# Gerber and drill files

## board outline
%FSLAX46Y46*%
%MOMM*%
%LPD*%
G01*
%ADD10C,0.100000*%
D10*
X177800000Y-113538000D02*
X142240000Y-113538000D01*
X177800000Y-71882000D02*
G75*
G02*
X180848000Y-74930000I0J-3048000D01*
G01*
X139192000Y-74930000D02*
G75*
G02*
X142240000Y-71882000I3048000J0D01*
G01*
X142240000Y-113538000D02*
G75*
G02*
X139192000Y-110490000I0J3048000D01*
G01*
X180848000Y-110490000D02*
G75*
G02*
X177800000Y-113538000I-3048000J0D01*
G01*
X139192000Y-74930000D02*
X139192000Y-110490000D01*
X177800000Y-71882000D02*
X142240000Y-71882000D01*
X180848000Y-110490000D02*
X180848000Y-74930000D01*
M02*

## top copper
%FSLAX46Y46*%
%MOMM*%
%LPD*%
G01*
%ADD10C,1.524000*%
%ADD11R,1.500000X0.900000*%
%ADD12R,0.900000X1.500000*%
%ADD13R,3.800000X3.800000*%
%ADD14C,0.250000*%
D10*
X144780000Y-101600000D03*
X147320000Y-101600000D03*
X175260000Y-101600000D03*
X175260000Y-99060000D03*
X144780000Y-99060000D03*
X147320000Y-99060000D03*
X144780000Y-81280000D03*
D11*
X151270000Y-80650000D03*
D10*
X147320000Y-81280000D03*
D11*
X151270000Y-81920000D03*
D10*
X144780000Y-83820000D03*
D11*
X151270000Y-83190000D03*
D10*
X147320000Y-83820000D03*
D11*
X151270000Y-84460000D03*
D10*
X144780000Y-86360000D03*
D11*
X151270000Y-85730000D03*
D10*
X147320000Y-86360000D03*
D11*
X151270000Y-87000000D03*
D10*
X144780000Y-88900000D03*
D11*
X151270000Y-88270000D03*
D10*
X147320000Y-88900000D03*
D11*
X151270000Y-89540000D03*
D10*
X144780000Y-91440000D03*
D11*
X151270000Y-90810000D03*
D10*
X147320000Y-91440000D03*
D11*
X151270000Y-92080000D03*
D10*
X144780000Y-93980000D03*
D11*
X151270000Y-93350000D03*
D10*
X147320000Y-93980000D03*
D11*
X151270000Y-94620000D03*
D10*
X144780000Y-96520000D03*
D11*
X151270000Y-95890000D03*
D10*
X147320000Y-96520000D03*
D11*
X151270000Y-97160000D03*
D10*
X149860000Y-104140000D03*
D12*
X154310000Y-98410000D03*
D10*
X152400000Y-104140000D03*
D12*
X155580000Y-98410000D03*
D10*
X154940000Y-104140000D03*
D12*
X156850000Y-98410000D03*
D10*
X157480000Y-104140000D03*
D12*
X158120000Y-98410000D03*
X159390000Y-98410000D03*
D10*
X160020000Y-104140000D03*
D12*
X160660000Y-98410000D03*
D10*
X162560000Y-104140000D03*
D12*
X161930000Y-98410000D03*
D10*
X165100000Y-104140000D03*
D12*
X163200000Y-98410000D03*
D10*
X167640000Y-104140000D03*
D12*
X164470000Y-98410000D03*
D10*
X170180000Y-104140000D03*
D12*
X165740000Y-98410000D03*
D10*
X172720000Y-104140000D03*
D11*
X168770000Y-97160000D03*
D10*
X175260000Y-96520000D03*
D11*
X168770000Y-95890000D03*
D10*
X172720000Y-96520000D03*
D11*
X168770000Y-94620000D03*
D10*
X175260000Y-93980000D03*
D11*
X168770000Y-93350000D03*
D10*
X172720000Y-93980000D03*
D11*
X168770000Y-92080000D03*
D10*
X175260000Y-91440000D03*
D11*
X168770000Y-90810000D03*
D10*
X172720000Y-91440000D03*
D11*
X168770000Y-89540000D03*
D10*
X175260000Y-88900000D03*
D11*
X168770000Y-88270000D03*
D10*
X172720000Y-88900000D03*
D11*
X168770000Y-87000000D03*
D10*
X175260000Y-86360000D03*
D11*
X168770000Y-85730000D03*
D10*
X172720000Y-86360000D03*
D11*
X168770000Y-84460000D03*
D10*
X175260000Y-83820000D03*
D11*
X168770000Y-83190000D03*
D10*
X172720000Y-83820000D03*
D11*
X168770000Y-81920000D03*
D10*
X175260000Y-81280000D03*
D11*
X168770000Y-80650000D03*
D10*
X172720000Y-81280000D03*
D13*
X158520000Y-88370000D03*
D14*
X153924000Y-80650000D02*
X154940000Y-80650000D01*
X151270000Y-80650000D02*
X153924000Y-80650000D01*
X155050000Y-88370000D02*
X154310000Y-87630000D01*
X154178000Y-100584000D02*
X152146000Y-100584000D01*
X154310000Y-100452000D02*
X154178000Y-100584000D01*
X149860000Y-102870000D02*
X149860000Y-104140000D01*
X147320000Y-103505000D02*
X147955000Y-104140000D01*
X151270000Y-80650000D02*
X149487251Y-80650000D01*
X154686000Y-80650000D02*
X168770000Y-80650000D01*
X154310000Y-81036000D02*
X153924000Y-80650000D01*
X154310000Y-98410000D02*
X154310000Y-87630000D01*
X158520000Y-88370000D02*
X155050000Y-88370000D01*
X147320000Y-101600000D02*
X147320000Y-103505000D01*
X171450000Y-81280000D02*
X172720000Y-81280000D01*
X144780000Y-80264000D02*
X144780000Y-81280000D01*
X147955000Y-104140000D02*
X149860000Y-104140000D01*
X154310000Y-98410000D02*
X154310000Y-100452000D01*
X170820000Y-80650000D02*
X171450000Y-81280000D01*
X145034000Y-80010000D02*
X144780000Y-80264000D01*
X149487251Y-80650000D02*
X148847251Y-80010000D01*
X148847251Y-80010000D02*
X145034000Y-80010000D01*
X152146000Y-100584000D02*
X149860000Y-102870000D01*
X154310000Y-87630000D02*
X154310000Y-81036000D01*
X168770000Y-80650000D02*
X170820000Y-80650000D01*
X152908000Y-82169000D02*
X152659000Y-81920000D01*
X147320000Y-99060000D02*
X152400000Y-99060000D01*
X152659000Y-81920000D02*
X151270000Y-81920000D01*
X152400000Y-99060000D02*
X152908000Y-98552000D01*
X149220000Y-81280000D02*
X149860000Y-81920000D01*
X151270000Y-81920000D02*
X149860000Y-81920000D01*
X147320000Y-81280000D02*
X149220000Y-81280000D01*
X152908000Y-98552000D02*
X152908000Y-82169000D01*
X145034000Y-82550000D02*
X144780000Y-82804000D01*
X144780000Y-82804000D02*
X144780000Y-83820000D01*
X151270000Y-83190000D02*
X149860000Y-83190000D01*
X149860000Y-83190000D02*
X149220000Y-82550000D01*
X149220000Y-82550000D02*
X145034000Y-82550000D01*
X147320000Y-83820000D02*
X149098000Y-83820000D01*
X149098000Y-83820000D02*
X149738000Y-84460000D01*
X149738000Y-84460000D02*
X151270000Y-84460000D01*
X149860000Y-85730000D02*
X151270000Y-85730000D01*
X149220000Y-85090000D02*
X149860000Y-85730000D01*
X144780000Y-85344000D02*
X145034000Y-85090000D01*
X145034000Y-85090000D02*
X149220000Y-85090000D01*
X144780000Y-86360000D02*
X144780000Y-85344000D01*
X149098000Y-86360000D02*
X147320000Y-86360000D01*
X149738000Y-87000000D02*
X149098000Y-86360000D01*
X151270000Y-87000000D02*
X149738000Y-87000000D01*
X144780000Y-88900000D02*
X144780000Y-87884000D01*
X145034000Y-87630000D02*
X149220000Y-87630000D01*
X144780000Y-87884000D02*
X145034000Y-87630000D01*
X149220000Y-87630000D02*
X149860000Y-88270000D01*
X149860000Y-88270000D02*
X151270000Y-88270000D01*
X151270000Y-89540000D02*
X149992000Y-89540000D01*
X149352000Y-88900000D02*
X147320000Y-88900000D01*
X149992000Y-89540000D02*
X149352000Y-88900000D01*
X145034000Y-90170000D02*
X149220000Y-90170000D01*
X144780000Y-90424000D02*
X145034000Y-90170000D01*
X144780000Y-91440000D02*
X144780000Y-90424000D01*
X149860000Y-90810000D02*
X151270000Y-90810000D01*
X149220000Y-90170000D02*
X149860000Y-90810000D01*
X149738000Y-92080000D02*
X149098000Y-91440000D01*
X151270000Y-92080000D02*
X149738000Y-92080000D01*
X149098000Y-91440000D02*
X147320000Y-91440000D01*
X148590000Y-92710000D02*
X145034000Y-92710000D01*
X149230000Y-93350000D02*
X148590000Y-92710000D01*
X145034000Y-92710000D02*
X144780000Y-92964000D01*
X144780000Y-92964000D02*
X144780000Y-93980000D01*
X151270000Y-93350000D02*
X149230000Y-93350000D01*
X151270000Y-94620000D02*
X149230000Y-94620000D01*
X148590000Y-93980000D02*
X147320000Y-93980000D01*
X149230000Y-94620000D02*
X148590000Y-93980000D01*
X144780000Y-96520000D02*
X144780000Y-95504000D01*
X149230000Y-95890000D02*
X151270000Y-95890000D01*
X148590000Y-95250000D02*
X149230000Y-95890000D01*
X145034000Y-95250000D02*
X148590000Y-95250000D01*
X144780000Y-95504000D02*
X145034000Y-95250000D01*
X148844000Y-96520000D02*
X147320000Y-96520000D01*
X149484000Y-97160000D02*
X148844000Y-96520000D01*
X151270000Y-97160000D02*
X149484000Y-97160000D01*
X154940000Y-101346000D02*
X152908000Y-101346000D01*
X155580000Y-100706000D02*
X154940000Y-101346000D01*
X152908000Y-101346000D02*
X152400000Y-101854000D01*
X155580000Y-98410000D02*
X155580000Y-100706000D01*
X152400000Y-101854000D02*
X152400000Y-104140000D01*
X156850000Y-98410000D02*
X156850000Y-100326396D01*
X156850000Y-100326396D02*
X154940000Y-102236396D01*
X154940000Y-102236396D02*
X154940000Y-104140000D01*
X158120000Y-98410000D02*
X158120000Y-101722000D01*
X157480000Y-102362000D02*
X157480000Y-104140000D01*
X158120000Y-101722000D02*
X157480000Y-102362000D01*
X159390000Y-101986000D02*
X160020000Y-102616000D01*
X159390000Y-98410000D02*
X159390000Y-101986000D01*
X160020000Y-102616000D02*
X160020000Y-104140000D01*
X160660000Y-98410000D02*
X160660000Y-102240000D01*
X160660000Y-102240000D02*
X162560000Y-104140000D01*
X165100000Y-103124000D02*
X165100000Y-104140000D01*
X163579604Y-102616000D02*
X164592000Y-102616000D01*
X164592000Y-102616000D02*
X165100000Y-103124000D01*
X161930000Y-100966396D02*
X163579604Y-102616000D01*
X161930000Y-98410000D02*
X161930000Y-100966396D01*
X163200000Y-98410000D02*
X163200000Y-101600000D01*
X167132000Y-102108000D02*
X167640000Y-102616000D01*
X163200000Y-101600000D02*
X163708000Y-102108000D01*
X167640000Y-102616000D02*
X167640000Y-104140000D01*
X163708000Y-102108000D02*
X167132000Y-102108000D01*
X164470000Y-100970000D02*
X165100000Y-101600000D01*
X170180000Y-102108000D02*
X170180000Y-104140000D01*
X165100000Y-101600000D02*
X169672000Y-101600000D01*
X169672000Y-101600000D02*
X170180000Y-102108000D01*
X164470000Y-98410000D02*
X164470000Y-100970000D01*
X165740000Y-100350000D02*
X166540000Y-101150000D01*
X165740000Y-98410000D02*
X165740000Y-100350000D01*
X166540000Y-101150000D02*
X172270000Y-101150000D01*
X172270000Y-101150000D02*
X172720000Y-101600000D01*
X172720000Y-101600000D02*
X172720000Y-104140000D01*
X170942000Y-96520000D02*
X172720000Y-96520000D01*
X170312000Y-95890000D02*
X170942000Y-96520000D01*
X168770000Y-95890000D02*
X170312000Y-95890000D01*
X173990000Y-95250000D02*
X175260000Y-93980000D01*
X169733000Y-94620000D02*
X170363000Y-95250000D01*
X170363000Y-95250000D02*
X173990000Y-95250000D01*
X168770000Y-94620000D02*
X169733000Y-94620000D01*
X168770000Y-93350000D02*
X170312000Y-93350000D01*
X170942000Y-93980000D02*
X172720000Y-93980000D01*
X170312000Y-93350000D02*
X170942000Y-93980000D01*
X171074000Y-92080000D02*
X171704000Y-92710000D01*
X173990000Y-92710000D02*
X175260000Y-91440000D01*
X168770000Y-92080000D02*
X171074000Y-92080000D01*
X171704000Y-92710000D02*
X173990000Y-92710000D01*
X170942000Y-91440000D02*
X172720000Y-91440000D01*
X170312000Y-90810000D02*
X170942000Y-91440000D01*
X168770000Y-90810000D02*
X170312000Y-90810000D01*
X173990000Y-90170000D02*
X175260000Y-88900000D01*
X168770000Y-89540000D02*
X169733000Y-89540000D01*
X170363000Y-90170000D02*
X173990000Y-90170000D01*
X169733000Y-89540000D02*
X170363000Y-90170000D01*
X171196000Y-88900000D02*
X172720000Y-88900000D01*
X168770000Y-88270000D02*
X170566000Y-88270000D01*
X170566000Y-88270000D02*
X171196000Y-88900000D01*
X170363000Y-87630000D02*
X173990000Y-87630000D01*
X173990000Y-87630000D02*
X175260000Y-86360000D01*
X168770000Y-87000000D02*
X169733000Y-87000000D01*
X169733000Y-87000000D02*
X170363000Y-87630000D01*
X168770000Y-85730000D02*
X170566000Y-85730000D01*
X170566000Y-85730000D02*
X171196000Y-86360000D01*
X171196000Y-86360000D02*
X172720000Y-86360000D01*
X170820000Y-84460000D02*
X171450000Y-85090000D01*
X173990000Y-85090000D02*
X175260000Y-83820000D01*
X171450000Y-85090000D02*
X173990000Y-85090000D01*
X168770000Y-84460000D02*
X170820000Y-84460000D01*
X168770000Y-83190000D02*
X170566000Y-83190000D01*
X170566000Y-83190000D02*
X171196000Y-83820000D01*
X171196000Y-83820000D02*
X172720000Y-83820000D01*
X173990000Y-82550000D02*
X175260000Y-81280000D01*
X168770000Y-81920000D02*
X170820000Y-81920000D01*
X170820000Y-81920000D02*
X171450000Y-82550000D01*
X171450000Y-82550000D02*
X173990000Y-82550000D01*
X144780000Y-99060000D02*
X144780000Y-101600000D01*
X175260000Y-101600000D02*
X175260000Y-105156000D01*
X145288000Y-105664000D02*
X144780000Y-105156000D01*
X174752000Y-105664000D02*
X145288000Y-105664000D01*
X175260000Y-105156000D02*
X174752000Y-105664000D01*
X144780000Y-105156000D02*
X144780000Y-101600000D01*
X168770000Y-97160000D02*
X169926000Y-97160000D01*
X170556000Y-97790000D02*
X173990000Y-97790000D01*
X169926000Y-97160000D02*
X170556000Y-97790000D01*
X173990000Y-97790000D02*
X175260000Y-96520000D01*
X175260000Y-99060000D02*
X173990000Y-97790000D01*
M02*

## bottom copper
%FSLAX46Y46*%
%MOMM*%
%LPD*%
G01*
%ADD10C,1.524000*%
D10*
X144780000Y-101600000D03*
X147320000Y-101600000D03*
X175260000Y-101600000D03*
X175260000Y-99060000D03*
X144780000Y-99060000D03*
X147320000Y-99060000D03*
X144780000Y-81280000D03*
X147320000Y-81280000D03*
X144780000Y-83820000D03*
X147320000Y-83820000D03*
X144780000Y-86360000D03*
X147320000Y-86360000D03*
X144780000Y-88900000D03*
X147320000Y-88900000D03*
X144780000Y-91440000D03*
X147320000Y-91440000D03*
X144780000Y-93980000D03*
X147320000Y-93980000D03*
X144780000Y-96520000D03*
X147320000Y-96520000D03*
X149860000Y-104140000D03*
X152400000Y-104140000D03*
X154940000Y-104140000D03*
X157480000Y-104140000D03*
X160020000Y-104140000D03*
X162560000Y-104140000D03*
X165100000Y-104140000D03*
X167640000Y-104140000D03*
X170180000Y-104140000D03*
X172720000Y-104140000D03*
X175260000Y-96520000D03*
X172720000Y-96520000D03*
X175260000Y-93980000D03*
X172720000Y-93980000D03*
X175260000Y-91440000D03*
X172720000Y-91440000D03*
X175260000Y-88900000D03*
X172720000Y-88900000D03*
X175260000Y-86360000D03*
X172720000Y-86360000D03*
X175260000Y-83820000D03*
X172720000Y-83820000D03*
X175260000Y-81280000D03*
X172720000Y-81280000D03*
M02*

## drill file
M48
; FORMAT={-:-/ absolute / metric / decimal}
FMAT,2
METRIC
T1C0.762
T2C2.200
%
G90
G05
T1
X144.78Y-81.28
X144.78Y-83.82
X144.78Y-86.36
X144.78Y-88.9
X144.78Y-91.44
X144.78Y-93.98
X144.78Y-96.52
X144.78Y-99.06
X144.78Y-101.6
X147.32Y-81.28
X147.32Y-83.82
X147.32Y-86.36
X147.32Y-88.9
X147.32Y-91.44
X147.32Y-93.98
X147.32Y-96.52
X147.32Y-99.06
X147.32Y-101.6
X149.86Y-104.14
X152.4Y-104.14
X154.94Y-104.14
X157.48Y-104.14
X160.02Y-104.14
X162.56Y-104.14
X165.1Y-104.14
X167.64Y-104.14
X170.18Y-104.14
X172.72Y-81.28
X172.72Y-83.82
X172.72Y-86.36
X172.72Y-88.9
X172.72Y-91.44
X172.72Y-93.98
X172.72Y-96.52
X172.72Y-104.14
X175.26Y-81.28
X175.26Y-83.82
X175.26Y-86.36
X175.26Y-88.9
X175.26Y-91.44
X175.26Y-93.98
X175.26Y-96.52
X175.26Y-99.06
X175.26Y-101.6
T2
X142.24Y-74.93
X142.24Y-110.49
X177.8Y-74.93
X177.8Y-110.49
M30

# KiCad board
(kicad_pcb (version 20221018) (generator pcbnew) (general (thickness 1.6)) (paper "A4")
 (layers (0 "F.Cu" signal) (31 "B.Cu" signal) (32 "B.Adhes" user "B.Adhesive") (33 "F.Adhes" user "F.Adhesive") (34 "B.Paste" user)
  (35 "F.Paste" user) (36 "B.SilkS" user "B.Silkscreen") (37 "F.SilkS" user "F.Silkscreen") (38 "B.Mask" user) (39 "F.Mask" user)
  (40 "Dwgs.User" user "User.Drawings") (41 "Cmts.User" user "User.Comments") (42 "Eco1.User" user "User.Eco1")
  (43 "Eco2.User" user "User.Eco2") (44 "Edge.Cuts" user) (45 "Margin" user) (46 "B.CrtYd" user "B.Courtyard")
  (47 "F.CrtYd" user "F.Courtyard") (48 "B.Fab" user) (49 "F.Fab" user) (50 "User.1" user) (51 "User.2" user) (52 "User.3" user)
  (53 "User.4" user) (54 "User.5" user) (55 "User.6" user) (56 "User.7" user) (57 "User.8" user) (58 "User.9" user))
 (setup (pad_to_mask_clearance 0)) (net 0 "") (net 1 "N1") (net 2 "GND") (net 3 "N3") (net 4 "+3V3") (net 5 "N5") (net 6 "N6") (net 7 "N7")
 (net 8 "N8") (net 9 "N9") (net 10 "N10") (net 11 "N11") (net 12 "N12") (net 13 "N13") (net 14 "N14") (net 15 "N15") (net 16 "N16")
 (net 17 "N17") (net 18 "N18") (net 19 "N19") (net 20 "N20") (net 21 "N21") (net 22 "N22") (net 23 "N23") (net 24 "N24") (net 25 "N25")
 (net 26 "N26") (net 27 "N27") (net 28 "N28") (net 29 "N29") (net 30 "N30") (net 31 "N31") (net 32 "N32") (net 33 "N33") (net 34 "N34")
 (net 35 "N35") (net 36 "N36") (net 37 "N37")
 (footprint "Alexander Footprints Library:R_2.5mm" (layer "F.Cu") (at 147.32 104.14)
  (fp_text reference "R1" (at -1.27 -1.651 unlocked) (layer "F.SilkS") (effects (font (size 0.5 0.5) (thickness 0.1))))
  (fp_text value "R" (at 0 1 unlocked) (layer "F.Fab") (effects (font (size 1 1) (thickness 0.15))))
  (pad "1" thru_hole circle (at -2.54 -2.54) (size 1.524 1.524) (drill 0.762) (layers "*.Cu" "*.Mask") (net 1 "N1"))
  (pad "2" thru_hole circle (at 0 -2.54) (size 1.524 1.524) (drill 0.762) (layers "*.Cu" "*.Mask") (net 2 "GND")))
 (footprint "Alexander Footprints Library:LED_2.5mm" (layer "F.Cu") (at 177.8 99.06 90)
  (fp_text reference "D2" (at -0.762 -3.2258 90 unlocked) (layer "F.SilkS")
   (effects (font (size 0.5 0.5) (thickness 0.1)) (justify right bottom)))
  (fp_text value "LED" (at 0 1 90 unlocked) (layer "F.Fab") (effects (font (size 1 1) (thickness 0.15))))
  (pad "1" thru_hole circle (at -2.54 -2.54 90) (size 1.524 1.524) (drill 0.762) (layers "*.Cu" "*.Mask") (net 1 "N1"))
  (pad "2" thru_hole circle (at 0 -2.54 90) (size 1.524 1.524) (drill 0.762) (layers "*.Cu" "*.Mask") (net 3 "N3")))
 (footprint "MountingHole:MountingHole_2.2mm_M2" (layer "F.Cu") (at 142.24 74.93)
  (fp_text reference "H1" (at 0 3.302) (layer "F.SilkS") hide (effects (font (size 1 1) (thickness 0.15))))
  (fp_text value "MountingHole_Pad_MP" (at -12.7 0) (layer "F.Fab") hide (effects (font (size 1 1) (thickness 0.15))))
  (pad "" np_thru_hole circle (at 0 0) (size 2.2 2.2) (drill 2.2) (layers "*.Cu" "*.Mask")))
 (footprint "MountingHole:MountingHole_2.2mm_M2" (layer "F.Cu") (at 142.24 110.49)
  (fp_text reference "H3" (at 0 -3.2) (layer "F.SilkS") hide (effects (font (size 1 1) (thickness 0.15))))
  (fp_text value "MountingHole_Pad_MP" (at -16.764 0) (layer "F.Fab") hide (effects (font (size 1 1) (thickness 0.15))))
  (pad "" np_thru_hole circle (at 0 0) (size 2.2 2.2) (drill 2.2) (layers "*.Cu" "*.Mask")))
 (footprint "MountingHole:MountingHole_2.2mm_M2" (layer "F.Cu") (at 177.8 110.49)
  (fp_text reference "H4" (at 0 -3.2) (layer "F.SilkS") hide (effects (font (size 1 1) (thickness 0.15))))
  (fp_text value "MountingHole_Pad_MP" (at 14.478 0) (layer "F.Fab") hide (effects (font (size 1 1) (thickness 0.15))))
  (pad "" np_thru_hole circle (at 0 0) (size 2.2 2.2) (drill 2.2) (layers "*.Cu" "*.Mask")))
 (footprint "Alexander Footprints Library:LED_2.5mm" (layer "F.Cu") (at 147.32 109.22)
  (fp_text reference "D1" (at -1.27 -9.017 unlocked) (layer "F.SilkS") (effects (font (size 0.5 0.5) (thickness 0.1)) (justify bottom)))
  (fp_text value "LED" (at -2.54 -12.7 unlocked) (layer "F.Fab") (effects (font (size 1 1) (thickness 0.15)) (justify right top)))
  (pad "1" thru_hole circle (at -2.54 -10.16) (size 1.524 1.524) (drill 0.762) (layers "*.Cu" "*.Mask") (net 1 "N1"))
  (pad "2" thru_hole circle (at 0 -10.16) (size 1.524 1.524) (drill 0.762) (layers "*.Cu" "*.Mask") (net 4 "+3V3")))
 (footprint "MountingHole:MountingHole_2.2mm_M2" (layer "F.Cu") (at 177.8 74.93)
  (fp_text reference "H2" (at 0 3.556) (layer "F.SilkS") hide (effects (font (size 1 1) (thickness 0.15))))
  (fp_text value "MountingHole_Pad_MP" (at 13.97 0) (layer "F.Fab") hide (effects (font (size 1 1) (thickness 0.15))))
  (pad "" np_thru_hole circle (at 0 0) (size 2.2 2.2) (drill 2.2) (layers "*.Cu" "*.Mask")))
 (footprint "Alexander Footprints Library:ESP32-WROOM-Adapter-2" (layer "F.Cu") (at 160.02 88.9)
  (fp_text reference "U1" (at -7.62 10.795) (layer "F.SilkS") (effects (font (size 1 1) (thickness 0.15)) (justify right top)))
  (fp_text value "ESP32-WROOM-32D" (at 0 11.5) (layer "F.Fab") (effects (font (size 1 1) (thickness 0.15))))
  (pad "1" thru_hole circle (at -15.24 -7.62) (size 1.524 1.524) (drill 0.762) (layers "*.Cu" "*.Mask") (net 2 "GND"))
  (pad "1" smd rect (at -8.75 -8.25) (size 1.5 0.9) (layers "F.Cu" "F.Paste" "F.Mask") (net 2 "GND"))
  (pad "2" thru_hole circle (at -12.7 -7.62) (size 1.524 1.524) (drill 0.762) (layers "*.Cu" "*.Mask") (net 4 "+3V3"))
  (pad "2" smd rect (at -8.75 -6.98) (size 1.5 0.9) (layers "F.Cu" "F.Paste" "F.Mask") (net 4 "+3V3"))
  (pad "3" thru_hole circle (at -15.24 -5.08) (size 1.524 1.524) (drill 0.762) (layers "*.Cu" "*.Mask") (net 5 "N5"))
  (pad "3" smd rect (at -8.75 -5.71) (size 1.5 0.9) (layers "F.Cu" "F.Paste" "F.Mask") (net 5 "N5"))
  (pad "4" thru_hole circle (at -12.7 -5.08) (size 1.524 1.524) (drill 0.762) (layers "*.Cu" "*.Mask") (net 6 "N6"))
  (pad "4" smd rect (at -8.75 -4.44) (size 1.5 0.9) (layers "F.Cu" "F.Paste" "F.Mask") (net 6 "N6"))
  (pad "5" thru_hole circle (at -15.24 -2.54) (size 1.524 1.524) (drill 0.762) (layers "*.Cu" "*.Mask") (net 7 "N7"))
  (pad "5" smd rect (at -8.75 -3.17) (size 1.5 0.9) (layers "F.Cu" "F.Paste" "F.Mask") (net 7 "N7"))
  (pad "6" thru_hole circle (at -12.7 -2.54) (size 1.524 1.524) (drill 0.762) (layers "*.Cu" "*.Mask") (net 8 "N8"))
  (pad "6" smd rect (at -8.75 -1.9) (size 1.5 0.9) (layers "F.Cu" "F.Paste" "F.Mask") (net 8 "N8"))
  (pad "7" thru_hole circle (at -15.24 0) (size 1.524 1.524) (drill 0.762) (layers "*.Cu" "*.Mask") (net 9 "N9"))
  (pad "7" smd rect (at -8.75 -0.63) (size 1.5 0.9) (layers "F.Cu" "F.Paste" "F.Mask") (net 9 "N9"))
  (pad "8" thru_hole circle (at -12.7 0) (size 1.524 1.524) (drill 0.762) (layers "*.Cu" "*.Mask") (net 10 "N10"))
  (pad "8" smd rect (at -8.75 0.64) (size 1.5 0.9) (layers "F.Cu" "F.Paste" "F.Mask") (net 10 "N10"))
  (pad "9" thru_hole circle (at -15.24 2.54) (size 1.524 1.524) (drill 0.762) (layers "*.Cu" "*.Mask") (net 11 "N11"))
  (pad "9" smd rect (at -8.75 1.91) (size 1.5 0.9) (layers "F.Cu" "F.Paste" "F.Mask") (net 11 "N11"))
  (pad "10" thru_hole circle (at -12.7 2.54) (size 1.524 1.524) (drill 0.762) (layers "*.Cu" "*.Mask") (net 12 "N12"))
  (pad "10" smd rect (at -8.75 3.18) (size 1.5 0.9) (layers "F.Cu" "F.Paste" "F.Mask") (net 12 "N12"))
  (pad "11" thru_hole circle (at -15.24 5.08) (size 1.524 1.524) (drill 0.762) (layers "*.Cu" "*.Mask") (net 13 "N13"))
  (pad "11" smd rect (at -8.75 4.45) (size 1.5 0.9) (layers "F.Cu" "F.Paste" "F.Mask") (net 13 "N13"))
  (pad "12" thru_hole circle (at -12.7 5.08) (size 1.524 1.524) (drill 0.762) (layers "*.Cu" "*.Mask") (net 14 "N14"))
  (pad "12" smd rect (at -8.75 5.72) (size 1.5 0.9) (layers "F.Cu" "F.Paste" "F.Mask") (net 14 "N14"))
  (pad "13" thru_hole circle (at -15.24 7.62) (size 1.524 1.524) (drill 0.762) (layers "*.Cu" "*.Mask") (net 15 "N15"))
  (pad "13" smd rect (at -8.75 6.99) (size 1.5 0.9) (layers "F.Cu" "F.Paste" "F.Mask") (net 15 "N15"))
  (pad "14" thru_hole circle (at -12.7 7.62) (size 1.524 1.524) (drill 0.762) (layers "*.Cu" "*.Mask") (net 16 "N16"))
  (pad "14" smd rect (at -8.75 8.26) (size 1.5 0.9) (layers "F.Cu" "F.Paste" "F.Mask") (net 16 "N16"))
  (pad "15" thru_hole circle (at -10.16 15.24 90) (size 1.524 1.524) (drill 0.762) (layers "*.Cu" "*.Mask") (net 2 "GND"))
  (pad "15" smd rect (at -5.71 9.51 90) (size 1.5 0.9) (layers "F.Cu" "F.Paste" "F.Mask") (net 2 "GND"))
  (pad "16" thru_hole circle (at -7.62 15.24 90) (size 1.524 1.524) (drill 0.762) (layers "*.Cu" "*.Mask") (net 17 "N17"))
  (pad "16" smd rect (at -4.44 9.51 90) (size 1.5 0.9) (layers "F.Cu" "F.Paste" "F.Mask") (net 17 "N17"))
  (pad "17" thru_hole circle (at -5.08 15.24 90) (size 1.524 1.524) (drill 0.762) (layers "*.Cu" "*.Mask") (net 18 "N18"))
  (pad "17" smd rect (at -3.17 9.51 90) (size 1.5 0.9) (layers "F.Cu" "F.Paste" "F.Mask") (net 18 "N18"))
  (pad "18" thru_hole circle (at -2.54 15.24 90) (size 1.524 1.524) (drill 0.762) (layers "*.Cu" "*.Mask") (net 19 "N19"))
  (pad "18" smd rect (at -1.9 9.51 90) (size 1.5 0.9) (layers "F.Cu" "F.Paste" "F.Mask") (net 19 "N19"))
  (pad "19" smd rect (at -0.63 9.51 90) (size 1.5 0.9) (layers "F.Cu" "F.Paste" "F.Mask") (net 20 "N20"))
  (pad "19" thru_hole circle (at 0 15.24 90) (size 1.524 1.524) (drill 0.762) (layers "*.Cu" "*.Mask") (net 20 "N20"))
  (pad "20" smd rect (at 0.64 9.51 90) (size 1.5 0.9) (layers "F.Cu" "F.Paste" "F.Mask") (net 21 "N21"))
  (pad "20" thru_hole circle (at 2.54 15.24 90) (size 1.524 1.524) (drill 0.762) (layers "*.Cu" "*.Mask") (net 21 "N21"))
  (pad "21" smd rect (at 1.91 9.51 90) (size 1.5 0.9) (layers "F.Cu" "F.Paste" "F.Mask") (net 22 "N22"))
  (pad "21" thru_hole circle (at 5.08 15.24 90) (size 1.524 1.524) (drill 0.762) (layers "*.Cu" "*.Mask") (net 22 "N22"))
  (pad "22" smd rect (at 3.18 9.51 90) (size 1.5 0.9) (layers "F.Cu" "F.Paste" "F.Mask") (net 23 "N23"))
  (pad "22" thru_hole circle (at 7.62 15.24 90) (size 1.524 1.524) (drill 0.762) (layers "*.Cu" "*.Mask") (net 23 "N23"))
  (pad "23" smd rect (at 4.45 9.51 90) (size 1.5 0.9) (layers "F.Cu" "F.Paste" "F.Mask") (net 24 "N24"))
  (pad "23" thru_hole circle (at 10.16 15.24 90) (size 1.524 1.524) (drill 0.762) (layers "*.Cu" "*.Mask") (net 24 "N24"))
  (pad "24" smd rect (at 5.72 9.51 90) (size 1.5 0.9) (layers "F.Cu" "F.Paste" "F.Mask") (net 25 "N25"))
  (pad "24" thru_hole circle (at 12.7 15.24 90) (size 1.524 1.524) (drill 0.762) (layers "*.Cu" "*.Mask") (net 25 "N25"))
  (pad "25" smd rect (at 8.75 8.26) (size 1.5 0.9) (layers "F.Cu" "F.Paste" "F.Mask") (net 3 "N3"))
  (pad "25" thru_hole circle (at 15.24 7.62) (size 1.524 1.524) (drill 0.762) (layers "*.Cu" "*.Mask") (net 3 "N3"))
  (pad "26" smd rect (at 8.75 6.99) (size 1.5 0.9) (layers "F.Cu" "F.Paste" "F.Mask") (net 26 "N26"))
  (pad "26" thru_hole circle (at 12.7 7.62) (size 1.524 1.524) (drill 0.762) (layers "*.Cu" "*.Mask") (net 26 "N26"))
  (pad "27" smd rect (at 8.75 5.72) (size 1.5 0.9) (layers "F.Cu" "F.Paste" "F.Mask") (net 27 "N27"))
  (pad "27" thru_hole circle (at 15.24 5.08) (size 1.524 1.524) (drill 0.762) (layers "*.Cu" "*.Mask") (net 27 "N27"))
  (pad "28" smd rect (at 8.75 4.45) (size 1.5 0.9) (layers "F.Cu" "F.Paste" "F.Mask") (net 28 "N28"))
  (pad "28" thru_hole circle (at 12.7 5.08) (size 1.524 1.524) (drill 0.762) (layers "*.Cu" "*.Mask") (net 28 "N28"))
  (pad "29" smd rect (at 8.75 3.18) (size 1.5 0.9) (layers "F.Cu" "F.Paste" "F.Mask") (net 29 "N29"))
  (pad "29" thru_hole circle (at 15.24 2.54) (size 1.524 1.524) (drill 0.762) (layers "*.Cu" "*.Mask") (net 29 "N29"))
  (pad "30" smd rect (at 8.75 1.91) (size 1.5 0.9) (layers "F.Cu" "F.Paste" "F.Mask") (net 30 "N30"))
  (pad "30" thru_hole circle (at 12.7 2.54) (size 1.524 1.524) (drill 0.762) (layers "*.Cu" "*.Mask") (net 30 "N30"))
  (pad "31" smd rect (at 8.75 0.64) (size 1.5 0.9) (layers "F.Cu" "F.Paste" "F.Mask") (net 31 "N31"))
  (pad "31" thru_hole circle (at 15.24 0) (size 1.524 1.524) (drill 0.762) (layers "*.Cu" "*.Mask") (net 31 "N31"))
  (pad "32" smd rect (at 8.75 -0.63) (size 1.5 0.9) (layers "F.Cu" "F.Paste" "F.Mask") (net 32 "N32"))
  (pad "32" thru_hole circle (at 12.7 0) (size 1.524 1.524) (drill 0.762) (layers "*.Cu" "*.Mask") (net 32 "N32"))
  (pad "33" smd rect (at 8.75 -1.9) (size 1.5 0.9) (layers "F.Cu" "F.Paste" "F.Mask") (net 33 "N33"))
  (pad "33" thru_hole circle (at 15.24 -2.54) (size 1.524 1.524) (drill 0.762) (layers "*.Cu" "*.Mask") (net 33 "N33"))
  (pad "34" smd rect (at 8.75 -3.17) (size 1.5 0.9) (layers "F.Cu" "F.Paste" "F.Mask") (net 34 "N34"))
  (pad "34" thru_hole circle (at 12.7 -2.54) (size 1.524 1.524) (drill 0.762) (layers "*.Cu" "*.Mask") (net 34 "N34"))
  (pad "35" smd rect (at 8.75 -4.44) (size 1.5 0.9) (layers "F.Cu" "F.Paste" "F.Mask") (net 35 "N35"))
  (pad "35" thru_hole circle (at 15.24 -5.08) (size 1.524 1.524) (drill 0.762) (layers "*.Cu" "*.Mask") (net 35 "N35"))
  (pad "36" smd rect (at 8.75 -5.71) (size 1.5 0.9) (layers "F.Cu" "F.Paste" "F.Mask") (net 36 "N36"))
  (pad "36" thru_hole circle (at 12.7 -5.08) (size 1.524 1.524) (drill 0.762) (layers "*.Cu" "*.Mask") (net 36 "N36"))
  (pad "37" smd rect (at 8.75 -6.98) (size 1.5 0.9) (layers "F.Cu" "F.Paste" "F.Mask") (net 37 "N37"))
  (pad "37" thru_hole circle (at 15.24 -7.62) (size 1.524 1.524) (drill 0.762) (layers "*.Cu" "*.Mask") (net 37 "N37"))
  (pad "38" smd rect (at 8.75 -8.25) (size 1.5 0.9) (layers "F.Cu" "F.Paste" "F.Mask") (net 2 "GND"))
  (pad "38" thru_hole circle (at 12.7 -7.62) (size 1.524 1.524) (drill 0.762) (layers "*.Cu" "*.Mask") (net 2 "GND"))
  (pad "39" smd rect (at -1.5 -0.53) (size 3.8 3.8) (layers "F.Cu" "F.Mask") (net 2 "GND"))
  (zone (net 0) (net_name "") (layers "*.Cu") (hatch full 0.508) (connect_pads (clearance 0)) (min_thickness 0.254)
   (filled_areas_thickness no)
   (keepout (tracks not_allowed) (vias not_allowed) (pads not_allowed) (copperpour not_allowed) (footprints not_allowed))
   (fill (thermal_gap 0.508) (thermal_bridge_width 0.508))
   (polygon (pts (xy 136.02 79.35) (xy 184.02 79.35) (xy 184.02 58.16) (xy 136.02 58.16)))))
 (gr_line (start 177.8 113.538) (end 142.24 113.538) (stroke (width 0.1) (type default)) (layer "Edge.Cuts"))
 (gr_arc (start 177.8 71.882) (mid 179.955261 72.774739) (end 180.848 74.93) (stroke (width 0.1) (type default)) (layer "Edge.Cuts"))
 (gr_arc (start 139.192 74.93) (mid 140.084739 72.774739) (end 142.24 71.882) (stroke (width 0.1) (type default)) (layer "Edge.Cuts"))
 (gr_arc (start 142.24 113.538) (mid 140.084739 112.645261) (end 139.192 110.49) (stroke (width 0.1) (type default)) (layer "Edge.Cuts"))
 (gr_arc (start 180.848 110.49) (mid 179.955261 112.645261) (end 177.8 113.538) (stroke (width 0.1) (type default)) (layer "Edge.Cuts"))
 (gr_line (start 139.192 74.93) (end 139.192 110.49) (stroke (width 0.1) (type default)) (layer "Edge.Cuts"))
 (gr_line (start 177.8 71.882) (end 142.24 71.882) (stroke (width 0.1) (type default)) (layer "Edge.Cuts"))
 (gr_line (start 180.848 110.49) (end 180.848 74.93) (stroke (width 0.1) (type default)) (layer "Edge.Cuts"))
 (segment (start 153.924 80.65) (end 154.94 80.65) (width 0.25) (layer "F.Cu") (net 2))
 (segment (start 151.27 80.65) (end 153.924 80.65) (width 0.25) (layer "F.Cu") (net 2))
 (segment (start 155.05 88.37) (end 154.31 87.63) (width 0.25) (layer "F.Cu") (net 2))
 (segment (start 154.178 100.584) (end 152.146 100.584) (width 0.25) (layer "F.Cu") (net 2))
 (segment (start 154.31 100.452) (end 154.178 100.584) (width 0.25) (layer "F.Cu") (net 2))
 (segment (start 149.86 102.87) (end 149.86 104.14) (width 0.25) (layer "F.Cu") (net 2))
 (segment (start 147.32 103.505) (end 147.955 104.14) (width 0.25) (layer "F.Cu") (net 2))
 (segment (start 151.27 80.65) (end 149.487251 80.65) (width 0.25) (layer "F.Cu") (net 2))
 (segment (start 154.686 80.65) (end 168.77 80.65) (width 0.25) (layer "F.Cu") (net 2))
 (segment (start 154.31 81.036) (end 153.924 80.65) (width 0.25) (layer "F.Cu") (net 2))
 (segment (start 154.31 98.41) (end 154.31 87.63) (width 0.25) (layer "F.Cu") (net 2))
 (segment (start 158.52 88.37) (end 155.05 88.37) (width 0.25) (layer "F.Cu") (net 2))
 (segment (start 147.32 101.6) (end 147.32 103.505) (width 0.25) (layer "F.Cu") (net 2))
 (segment (start 171.45 81.28) (end 172.72 81.28) (width 0.25) (layer "F.Cu") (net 2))
 (segment (start 144.78 80.264) (end 144.78 81.28) (width 0.25) (layer "F.Cu") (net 2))
 (segment (start 147.955 104.14) (end 149.86 104.14) (width 0.25) (layer "F.Cu") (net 2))
 (segment (start 154.31 98.41) (end 154.31 100.452) (width 0.25) (layer "F.Cu") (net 2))
 (segment (start 170.82 80.65) (end 171.45 81.28) (width 0.25) (layer "F.Cu") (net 2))
 (segment (start 145.034 80.01) (end 144.78 80.264) (width 0.25) (layer "F.Cu") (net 2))
 (segment (start 149.487251 80.65) (end 148.847251 80.01) (width 0.25) (layer "F.Cu") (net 2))
 (segment (start 148.847251 80.01) (end 145.034 80.01) (width 0.25) (layer "F.Cu") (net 2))
 (segment (start 152.146 100.584) (end 149.86 102.87) (width 0.25) (layer "F.Cu") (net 2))
 (segment (start 154.31 87.63) (end 154.31 81.036) (width 0.25) (layer "F.Cu") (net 2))
 (segment (start 168.77 80.65) (end 170.82 80.65) (width 0.25) (layer "F.Cu") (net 2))
 (segment (start 152.908 82.169) (end 152.659 81.92) (width 0.25) (layer "F.Cu") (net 4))
 (segment (start 147.32 99.06) (end 152.4 99.06) (width 0.25) (layer "F.Cu") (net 4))
 (segment (start 152.659 81.92) (end 151.27 81.92) (width 0.25) (layer "F.Cu") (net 4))
 (segment (start 152.4 99.06) (end 152.908 98.552) (width 0.25) (layer "F.Cu") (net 4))
 (segment (start 149.22 81.28) (end 149.86 81.92) (width 0.25) (layer "F.Cu") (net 4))
 (segment (start 151.27 81.92) (end 149.86 81.92) (width 0.25) (layer "F.Cu") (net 4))
 (segment (start 147.32 81.28) (end 149.22 81.28) (width 0.25) (layer "F.Cu") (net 4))
 (segment (start 152.908 98.552) (end 152.908 82.169) (width 0.25) (layer "F.Cu") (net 4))
 (segment (start 145.034 82.55) (end 144.78 82.804) (width 0.25) (layer "F.Cu") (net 5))
 (segment (start 144.78 82.804) (end 144.78 83.82) (width 0.25) (layer "F.Cu") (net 5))
 (segment (start 151.27 83.19) (end 149.86 83.19) (width 0.25) (layer "F.Cu") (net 5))
 (segment (start 149.86 83.19) (end 149.22 82.55) (width 0.25) (layer "F.Cu") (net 5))
 (segment (start 149.22 82.55) (end 145.034 82.55) (width 0.25) (layer "F.Cu") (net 5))
 (segment (start 147.32 83.82) (end 149.098 83.82) (width 0.25) (layer "F.Cu") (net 6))
 (segment (start 149.098 83.82) (end 149.738 84.46) (width 0.25) (layer "F.Cu") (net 6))
 (segment (start 149.738 84.46) (end 151.27 84.46) (width 0.25) (layer "F.Cu") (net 6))
 (segment (start 149.86 85.73) (end 151.27 85.73) (width 0.25) (layer "F.Cu") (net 7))
 (segment (start 149.22 85.09) (end 149.86 85.73) (width 0.25) (layer "F.Cu") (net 7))
 (segment (start 144.78 85.344) (end 145.034 85.09) (width 0.25) (layer "F.Cu") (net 7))
 (segment (start 145.034 85.09) (end 149.22 85.09) (width 0.25) (layer "F.Cu") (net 7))
 (segment (start 144.78 86.36) (end 144.78 85.344) (width 0.25) (layer "F.Cu") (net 7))
 (segment (start 149.098 86.36) (end 147.32 86.36) (width 0.25) (layer "F.Cu") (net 8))
 (segment (start 149.738 87) (end 149.098 86.36) (width 0.25) (layer "F.Cu") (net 8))
 (segment (start 151.27 87) (end 149.738 87) (width 0.25) (layer "F.Cu") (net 8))
 (segment (start 144.78 88.9) (end 144.78 87.884) (width 0.25) (layer "F.Cu") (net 9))
 (segment (start 145.034 87.63) (end 149.22 87.63) (width 0.25) (layer "F.Cu") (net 9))
 (segment (start 144.78 87.884) (end 145.034 87.63) (width 0.25) (layer "F.Cu") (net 9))
 (segment (start 149.22 87.63) (end 149.86 88.27) (width 0.25) (layer "F.Cu") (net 9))
 (segment (start 149.86 88.27) (end 151.27 88.27) (width 0.25) (layer "F.Cu") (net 9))
 (segment (start 151.27 89.54) (end 149.992 89.54) (width 0.25) (layer "F.Cu") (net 10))
 (segment (start 149.352 88.9) (end 147.32 88.9) (width 0.25) (layer "F.Cu") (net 10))
 (segment (start 149.992 89.54) (end 149.352 88.9) (width 0.25) (layer "F.Cu") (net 10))
 (segment (start 145.034 90.17) (end 149.22 90.17) (width 0.25) (layer "F.Cu") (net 11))
 (segment (start 144.78 90.424) (end 145.034 90.17) (width 0.25) (layer "F.Cu") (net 11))
 (segment (start 144.78 91.44) (end 144.78 90.424) (width 0.25) (layer "F.Cu") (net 11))
 (segment (start 149.86 90.81) (end 151.27 90.81) (width 0.25) (layer "F.Cu") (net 11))
 (segment (start 149.22 90.17) (end 149.86 90.81) (width 0.25) (layer "F.Cu") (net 11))
 (segment (start 149.738 92.08) (end 149.098 91.44) (width 0.25) (layer "F.Cu") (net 12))
 (segment (start 151.27 92.08) (end 149.738 92.08) (width 0.25) (layer "F.Cu") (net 12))
 (segment (start 149.098 91.44) (end 147.32 91.44) (width 0.25) (layer "F.Cu") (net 12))
 (segment (start 148.59 92.71) (end 145.034 92.71) (width 0.25) (layer "F.Cu") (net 13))
 (segment (start 149.23 93.35) (end 148.59 92.71) (width 0.25) (layer "F.Cu") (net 13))
 (segment (start 145.034 92.71) (end 144.78 92.964) (width 0.25) (layer "F.Cu") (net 13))
 (segment (start 144.78 92.964) (end 144.78 93.98) (width 0.25) (layer "F.Cu") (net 13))
 (segment (start 151.27 93.35) (end 149.23 93.35) (width 0.25) (layer "F.Cu") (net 13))
 (segment (start 151.27 94.62) (end 149.23 94.62) (width 0.25) (layer "F.Cu") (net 14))
 (segment (start 148.59 93.98) (end 147.32 93.98) (width 0.25) (layer "F.Cu") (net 14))
 (segment (start 149.23 94.62) (end 148.59 93.98) (width 0.25) (layer "F.Cu") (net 14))
 (segment (start 144.78 96.52) (end 144.78 95.504) (width 0.25) (layer "F.Cu") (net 15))
 (segment (start 149.23 95.89) (end 151.27 95.89) (width 0.25) (layer "F.Cu") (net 15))
 (segment (start 148.59 95.25) (end 149.23 95.89) (width 0.25) (layer "F.Cu") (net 15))
 (segment (start 145.034 95.25) (end 148.59 95.25) (width 0.25) (layer "F.Cu") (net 15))
 (segment (start 144.78 95.504) (end 145.034 95.25) (width 0.25) (layer "F.Cu") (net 15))
 (segment (start 148.844 96.52) (end 147.32 96.52) (width 0.25) (layer "F.Cu") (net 16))
 (segment (start 149.484 97.16) (end 148.844 96.52) (width 0.25) (layer "F.Cu") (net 16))
 (segment (start 151.27 97.16) (end 149.484 97.16) (width 0.25) (layer "F.Cu") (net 16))
 (segment (start 154.94 101.346) (end 152.908 101.346) (width 0.25) (layer "F.Cu") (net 17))
 (segment (start 155.58 100.706) (end 154.94 101.346) (width 0.25) (layer "F.Cu") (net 17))
 (segment (start 152.908 101.346) (end 152.4 101.854) (width 0.25) (layer "F.Cu") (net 17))
 (segment (start 155.58 98.41) (end 155.58 100.706) (width 0.25) (layer "F.Cu") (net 17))
 (segment (start 152.4 101.854) (end 152.4 104.14) (width 0.25) (layer "F.Cu") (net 17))
 (segment (start 156.85 98.41) (end 156.85 100.326396) (width 0.25) (layer "F.Cu") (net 18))
 (segment (start 156.85 100.326396) (end 154.94 102.236396) (width 0.25) (layer "F.Cu") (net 18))
 (segment (start 154.94 102.236396) (end 154.94 104.14) (width 0.25) (layer "F.Cu") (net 18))
 (segment (start 158.12 98.41) (end 158.12 101.722) (width 0.25) (layer "F.Cu") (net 19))
 (segment (start 157.48 102.362) (end 157.48 104.14) (width 0.25) (layer "F.Cu") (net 19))
 (segment (start 158.12 101.722) (end 157.48 102.362) (width 0.25) (layer "F.Cu") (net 19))
 (segment (start 159.39 101.986) (end 160.02 102.616) (width 0.25) (layer "F.Cu") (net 20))
 (segment (start 159.39 98.41) (end 159.39 101.986) (width 0.25) (layer "F.Cu") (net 20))
 (segment (start 160.02 102.616) (end 160.02 104.14) (width 0.25) (layer "F.Cu") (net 20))
 (segment (start 160.66 98.41) (end 160.66 102.24) (width 0.25) (layer "F.Cu") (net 21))
 (segment (start 160.66 102.24) (end 162.56 104.14) (width 0.25) (layer "F.Cu") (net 21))
 (segment (start 165.1 103.124) (end 165.1 104.14) (width 0.25) (layer "F.Cu") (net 22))
 (segment (start 163.579604 102.616) (end 164.592 102.616) (width 0.25) (layer "F.Cu") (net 22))
 (segment (start 164.592 102.616) (end 165.1 103.124) (width 0.25) (layer "F.Cu") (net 22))
 (segment (start 161.93 100.966396) (end 163.579604 102.616) (width 0.25) (layer "F.Cu") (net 22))
 (segment (start 161.93 98.41) (end 161.93 100.966396) (width 0.25) (layer "F.Cu") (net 22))
 (segment (start 163.2 98.41) (end 163.2 101.6) (width 0.25) (layer "F.Cu") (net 23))
 (segment (start 167.132 102.108) (end 167.64 102.616) (width 0.25) (layer "F.Cu") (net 23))
 (segment (start 163.2 101.6) (end 163.708 102.108) (width 0.25) (layer "F.Cu") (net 23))
 (segment (start 167.64 102.616) (end 167.64 104.14) (width 0.25) (layer "F.Cu") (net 23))
 (segment (start 163.708 102.108) (end 167.132 102.108) (width 0.25) (layer "F.Cu") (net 23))
 (segment (start 164.47 100.97) (end 165.1 101.6) (width 0.25) (layer "F.Cu") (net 24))
 (segment (start 170.18 102.108) (end 170.18 104.14) (width 0.25) (layer "F.Cu") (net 24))
 (segment (start 165.1 101.6) (end 169.672 101.6) (width 0.25) (layer "F.Cu") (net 24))
 (segment (start 169.672 101.6) (end 170.18 102.108) (width 0.25) (layer "F.Cu") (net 24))
 (segment (start 164.47 98.41) (end 164.47 100.97) (width 0.25) (layer "F.Cu") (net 24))
 (segment (start 165.74 100.35) (end 166.54 101.15) (width 0.25) (layer "F.Cu") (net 25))
 (segment (start 165.74 98.41) (end 165.74 100.35) (width 0.25) (layer "F.Cu") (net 25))
 (segment (start 166.54 101.15) (end 172.27 101.15) (width 0.25) (layer "F.Cu") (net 25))
 (segment (start 172.27 101.15) (end 172.72 101.6) (width 0.25) (layer "F.Cu") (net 25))
 (segment (start 172.72 101.6) (end 172.72 104.14) (width 0.25) (layer "F.Cu") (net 25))
 (segment (start 170.942 96.52) (end 172.72 96.52) (width 0.25) (layer "F.Cu") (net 26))
 (segment (start 170.312 95.89) (end 170.942 96.52) (width 0.25) (layer "F.Cu") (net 26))
 (segment (start 168.77 95.89) (end 170.312 95.89) (width 0.25) (layer "F.Cu") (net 26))
 (segment (start 173.99 95.25) (end 175.26 93.98) (width 0.25) (layer "F.Cu") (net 27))
 (segment (start 169.733 94.62) (end 170.363 95.25) (width 0.25) (layer "F.Cu") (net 27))
 (segment (start 170.363 95.25) (end 173.99 95.25) (width 0.25) (layer "F.Cu") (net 27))
 (segment (start 168.77 94.62) (end 169.733 94.62) (width 0.25) (layer "F.Cu") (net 27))
 (segment (start 168.77 93.35) (end 170.312 93.35) (width 0.25) (layer "F.Cu") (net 28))
 (segment (start 170.942 93.98) (end 172.72 93.98) (width 0.25) (layer "F.Cu") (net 28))
 (segment (start 170.312 93.35) (end 170.942 93.98) (width 0.25) (layer "F.Cu") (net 28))
 (segment (start 171.074 92.08) (end 171.704 92.71) (width 0.25) (layer "F.Cu") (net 29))
 (segment (start 173.99 92.71) (end 175.26 91.44) (width 0.25) (layer "F.Cu") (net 29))
 (segment (start 168.77 92.08) (end 171.074 92.08) (width 0.25) (layer "F.Cu") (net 29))
 (segment (start 171.704 92.71) (end 173.99 92.71) (width 0.25) (layer "F.Cu") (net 29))
 (segment (start 170.942 91.44) (end 172.72 91.44) (width 0.25) (layer "F.Cu") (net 30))
 (segment (start 170.312 90.81) (end 170.942 91.44) (width 0.25) (layer "F.Cu") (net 30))
 (segment (start 168.77 90.81) (end 170.312 90.81) (width 0.25) (layer "F.Cu") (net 30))
 (segment (start 173.99 90.17) (end 175.26 88.9) (width 0.25) (layer "F.Cu") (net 31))
 (segment (start 168.77 89.54) (end 169.733 89.54) (width 0.25) (layer "F.Cu") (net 31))
 (segment (start 170.363 90.17) (end 173.99 90.17) (width 0.25) (layer "F.Cu") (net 31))
 (segment (start 169.733 89.54) (end 170.363 90.17) (width 0.25) (layer "F.Cu") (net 31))
 (segment (start 171.196 88.9) (end 172.72 88.9) (width 0.25) (layer "F.Cu") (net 32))
 (segment (start 168.77 88.27) (end 170.566 88.27) (width 0.25) (layer "F.Cu") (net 32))
 (segment (start 170.566 88.27) (end 171.196 88.9) (width 0.25) (layer "F.Cu") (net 32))
 (segment (start 170.363 87.63) (end 173.99 87.63) (width 0.25) (layer "F.Cu") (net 33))
 (segment (start 173.99 87.63) (end 175.26 86.36) (width 0.25) (layer "F.Cu") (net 33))
 (segment (start 168.77 87) (end 169.733 87) (width 0.25) (layer "F.Cu") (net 33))
 (segment (start 169.733 87) (end 170.363 87.63) (width 0.25) (layer "F.Cu") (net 33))
 (segment (start 168.77 85.73) (end 170.566 85.73) (width 0.25) (layer "F.Cu") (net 34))
 (segment (start 170.566 85.73) (end 171.196 86.36) (width 0.25) (layer "F.Cu") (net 34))
 (segment (start 171.196 86.36) (end 172.72 86.36) (width 0.25) (layer "F.Cu") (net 34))
 (segment (start 170.82 84.46) (end 171.45 85.09) (width 0.25) (layer "F.Cu") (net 35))
 (segment (start 173.99 85.09) (end 175.26 83.82) (width 0.25) (layer "F.Cu") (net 35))
 (segment (start 171.45 85.09) (end 173.99 85.09) (width 0.25) (layer "F.Cu") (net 35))
 (segment (start 168.77 84.46) (end 170.82 84.46) (width 0.25) (layer "F.Cu") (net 35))
 (segment (start 168.77 83.19) (end 170.566 83.19) (width 0.25) (layer "F.Cu") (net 36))
 (segment (start 170.566 83.19) (end 171.196 83.82) (width 0.25) (layer "F.Cu") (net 36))
 (segment (start 171.196 83.82) (end 172.72 83.82) (width 0.25) (layer "F.Cu") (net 36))
 (segment (start 173.99 82.55) (end 175.26 81.28) (width 0.25) (layer "F.Cu") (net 37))
 (segment (start 168.77 81.92) (end 170.82 81.92) (width 0.25) (layer "F.Cu") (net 37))
 (segment (start 170.82 81.92) (end 171.45 82.55) (width 0.25) (layer "F.Cu") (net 37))
 (segment (start 171.45 82.55) (end 173.99 82.55) (width 0.25) (layer "F.Cu") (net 37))
 (segment (start 144.78 99.06) (end 144.78 101.6) (width 0.25) (layer "F.Cu") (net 1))
 (segment (start 175.26 101.6) (end 175.26 105.156) (width 0.25) (layer "F.Cu") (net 1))
 (segment (start 145.288 105.664) (end 144.78 105.156) (width 0.25) (layer "F.Cu") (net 1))
 (segment (start 174.752 105.664) (end 145.288 105.664) (width 0.25) (layer "F.Cu") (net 1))
 (segment (start 175.26 105.156) (end 174.752 105.664) (width 0.25) (layer "F.Cu") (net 1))
 (segment (start 144.78 105.156) (end 144.78 101.6) (width 0.25) (layer "F.Cu") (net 1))
 (segment (start 168.77 97.16) (end 169.926 97.16) (width 0.25) (layer "F.Cu") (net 3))
 (segment (start 170.556 97.79) (end 173.99 97.79) (width 0.25) (layer "F.Cu") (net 3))
 (segment (start 169.926 97.16) (end 170.556 97.79) (width 0.25) (layer "F.Cu") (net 3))
 (segment (start 173.99 97.79) (end 175.26 96.52) (width 0.25) (layer "F.Cu") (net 3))
 (segment (start 175.26 99.06) (end 173.99 97.79) (width 0.25) (layer "F.Cu") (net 3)))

